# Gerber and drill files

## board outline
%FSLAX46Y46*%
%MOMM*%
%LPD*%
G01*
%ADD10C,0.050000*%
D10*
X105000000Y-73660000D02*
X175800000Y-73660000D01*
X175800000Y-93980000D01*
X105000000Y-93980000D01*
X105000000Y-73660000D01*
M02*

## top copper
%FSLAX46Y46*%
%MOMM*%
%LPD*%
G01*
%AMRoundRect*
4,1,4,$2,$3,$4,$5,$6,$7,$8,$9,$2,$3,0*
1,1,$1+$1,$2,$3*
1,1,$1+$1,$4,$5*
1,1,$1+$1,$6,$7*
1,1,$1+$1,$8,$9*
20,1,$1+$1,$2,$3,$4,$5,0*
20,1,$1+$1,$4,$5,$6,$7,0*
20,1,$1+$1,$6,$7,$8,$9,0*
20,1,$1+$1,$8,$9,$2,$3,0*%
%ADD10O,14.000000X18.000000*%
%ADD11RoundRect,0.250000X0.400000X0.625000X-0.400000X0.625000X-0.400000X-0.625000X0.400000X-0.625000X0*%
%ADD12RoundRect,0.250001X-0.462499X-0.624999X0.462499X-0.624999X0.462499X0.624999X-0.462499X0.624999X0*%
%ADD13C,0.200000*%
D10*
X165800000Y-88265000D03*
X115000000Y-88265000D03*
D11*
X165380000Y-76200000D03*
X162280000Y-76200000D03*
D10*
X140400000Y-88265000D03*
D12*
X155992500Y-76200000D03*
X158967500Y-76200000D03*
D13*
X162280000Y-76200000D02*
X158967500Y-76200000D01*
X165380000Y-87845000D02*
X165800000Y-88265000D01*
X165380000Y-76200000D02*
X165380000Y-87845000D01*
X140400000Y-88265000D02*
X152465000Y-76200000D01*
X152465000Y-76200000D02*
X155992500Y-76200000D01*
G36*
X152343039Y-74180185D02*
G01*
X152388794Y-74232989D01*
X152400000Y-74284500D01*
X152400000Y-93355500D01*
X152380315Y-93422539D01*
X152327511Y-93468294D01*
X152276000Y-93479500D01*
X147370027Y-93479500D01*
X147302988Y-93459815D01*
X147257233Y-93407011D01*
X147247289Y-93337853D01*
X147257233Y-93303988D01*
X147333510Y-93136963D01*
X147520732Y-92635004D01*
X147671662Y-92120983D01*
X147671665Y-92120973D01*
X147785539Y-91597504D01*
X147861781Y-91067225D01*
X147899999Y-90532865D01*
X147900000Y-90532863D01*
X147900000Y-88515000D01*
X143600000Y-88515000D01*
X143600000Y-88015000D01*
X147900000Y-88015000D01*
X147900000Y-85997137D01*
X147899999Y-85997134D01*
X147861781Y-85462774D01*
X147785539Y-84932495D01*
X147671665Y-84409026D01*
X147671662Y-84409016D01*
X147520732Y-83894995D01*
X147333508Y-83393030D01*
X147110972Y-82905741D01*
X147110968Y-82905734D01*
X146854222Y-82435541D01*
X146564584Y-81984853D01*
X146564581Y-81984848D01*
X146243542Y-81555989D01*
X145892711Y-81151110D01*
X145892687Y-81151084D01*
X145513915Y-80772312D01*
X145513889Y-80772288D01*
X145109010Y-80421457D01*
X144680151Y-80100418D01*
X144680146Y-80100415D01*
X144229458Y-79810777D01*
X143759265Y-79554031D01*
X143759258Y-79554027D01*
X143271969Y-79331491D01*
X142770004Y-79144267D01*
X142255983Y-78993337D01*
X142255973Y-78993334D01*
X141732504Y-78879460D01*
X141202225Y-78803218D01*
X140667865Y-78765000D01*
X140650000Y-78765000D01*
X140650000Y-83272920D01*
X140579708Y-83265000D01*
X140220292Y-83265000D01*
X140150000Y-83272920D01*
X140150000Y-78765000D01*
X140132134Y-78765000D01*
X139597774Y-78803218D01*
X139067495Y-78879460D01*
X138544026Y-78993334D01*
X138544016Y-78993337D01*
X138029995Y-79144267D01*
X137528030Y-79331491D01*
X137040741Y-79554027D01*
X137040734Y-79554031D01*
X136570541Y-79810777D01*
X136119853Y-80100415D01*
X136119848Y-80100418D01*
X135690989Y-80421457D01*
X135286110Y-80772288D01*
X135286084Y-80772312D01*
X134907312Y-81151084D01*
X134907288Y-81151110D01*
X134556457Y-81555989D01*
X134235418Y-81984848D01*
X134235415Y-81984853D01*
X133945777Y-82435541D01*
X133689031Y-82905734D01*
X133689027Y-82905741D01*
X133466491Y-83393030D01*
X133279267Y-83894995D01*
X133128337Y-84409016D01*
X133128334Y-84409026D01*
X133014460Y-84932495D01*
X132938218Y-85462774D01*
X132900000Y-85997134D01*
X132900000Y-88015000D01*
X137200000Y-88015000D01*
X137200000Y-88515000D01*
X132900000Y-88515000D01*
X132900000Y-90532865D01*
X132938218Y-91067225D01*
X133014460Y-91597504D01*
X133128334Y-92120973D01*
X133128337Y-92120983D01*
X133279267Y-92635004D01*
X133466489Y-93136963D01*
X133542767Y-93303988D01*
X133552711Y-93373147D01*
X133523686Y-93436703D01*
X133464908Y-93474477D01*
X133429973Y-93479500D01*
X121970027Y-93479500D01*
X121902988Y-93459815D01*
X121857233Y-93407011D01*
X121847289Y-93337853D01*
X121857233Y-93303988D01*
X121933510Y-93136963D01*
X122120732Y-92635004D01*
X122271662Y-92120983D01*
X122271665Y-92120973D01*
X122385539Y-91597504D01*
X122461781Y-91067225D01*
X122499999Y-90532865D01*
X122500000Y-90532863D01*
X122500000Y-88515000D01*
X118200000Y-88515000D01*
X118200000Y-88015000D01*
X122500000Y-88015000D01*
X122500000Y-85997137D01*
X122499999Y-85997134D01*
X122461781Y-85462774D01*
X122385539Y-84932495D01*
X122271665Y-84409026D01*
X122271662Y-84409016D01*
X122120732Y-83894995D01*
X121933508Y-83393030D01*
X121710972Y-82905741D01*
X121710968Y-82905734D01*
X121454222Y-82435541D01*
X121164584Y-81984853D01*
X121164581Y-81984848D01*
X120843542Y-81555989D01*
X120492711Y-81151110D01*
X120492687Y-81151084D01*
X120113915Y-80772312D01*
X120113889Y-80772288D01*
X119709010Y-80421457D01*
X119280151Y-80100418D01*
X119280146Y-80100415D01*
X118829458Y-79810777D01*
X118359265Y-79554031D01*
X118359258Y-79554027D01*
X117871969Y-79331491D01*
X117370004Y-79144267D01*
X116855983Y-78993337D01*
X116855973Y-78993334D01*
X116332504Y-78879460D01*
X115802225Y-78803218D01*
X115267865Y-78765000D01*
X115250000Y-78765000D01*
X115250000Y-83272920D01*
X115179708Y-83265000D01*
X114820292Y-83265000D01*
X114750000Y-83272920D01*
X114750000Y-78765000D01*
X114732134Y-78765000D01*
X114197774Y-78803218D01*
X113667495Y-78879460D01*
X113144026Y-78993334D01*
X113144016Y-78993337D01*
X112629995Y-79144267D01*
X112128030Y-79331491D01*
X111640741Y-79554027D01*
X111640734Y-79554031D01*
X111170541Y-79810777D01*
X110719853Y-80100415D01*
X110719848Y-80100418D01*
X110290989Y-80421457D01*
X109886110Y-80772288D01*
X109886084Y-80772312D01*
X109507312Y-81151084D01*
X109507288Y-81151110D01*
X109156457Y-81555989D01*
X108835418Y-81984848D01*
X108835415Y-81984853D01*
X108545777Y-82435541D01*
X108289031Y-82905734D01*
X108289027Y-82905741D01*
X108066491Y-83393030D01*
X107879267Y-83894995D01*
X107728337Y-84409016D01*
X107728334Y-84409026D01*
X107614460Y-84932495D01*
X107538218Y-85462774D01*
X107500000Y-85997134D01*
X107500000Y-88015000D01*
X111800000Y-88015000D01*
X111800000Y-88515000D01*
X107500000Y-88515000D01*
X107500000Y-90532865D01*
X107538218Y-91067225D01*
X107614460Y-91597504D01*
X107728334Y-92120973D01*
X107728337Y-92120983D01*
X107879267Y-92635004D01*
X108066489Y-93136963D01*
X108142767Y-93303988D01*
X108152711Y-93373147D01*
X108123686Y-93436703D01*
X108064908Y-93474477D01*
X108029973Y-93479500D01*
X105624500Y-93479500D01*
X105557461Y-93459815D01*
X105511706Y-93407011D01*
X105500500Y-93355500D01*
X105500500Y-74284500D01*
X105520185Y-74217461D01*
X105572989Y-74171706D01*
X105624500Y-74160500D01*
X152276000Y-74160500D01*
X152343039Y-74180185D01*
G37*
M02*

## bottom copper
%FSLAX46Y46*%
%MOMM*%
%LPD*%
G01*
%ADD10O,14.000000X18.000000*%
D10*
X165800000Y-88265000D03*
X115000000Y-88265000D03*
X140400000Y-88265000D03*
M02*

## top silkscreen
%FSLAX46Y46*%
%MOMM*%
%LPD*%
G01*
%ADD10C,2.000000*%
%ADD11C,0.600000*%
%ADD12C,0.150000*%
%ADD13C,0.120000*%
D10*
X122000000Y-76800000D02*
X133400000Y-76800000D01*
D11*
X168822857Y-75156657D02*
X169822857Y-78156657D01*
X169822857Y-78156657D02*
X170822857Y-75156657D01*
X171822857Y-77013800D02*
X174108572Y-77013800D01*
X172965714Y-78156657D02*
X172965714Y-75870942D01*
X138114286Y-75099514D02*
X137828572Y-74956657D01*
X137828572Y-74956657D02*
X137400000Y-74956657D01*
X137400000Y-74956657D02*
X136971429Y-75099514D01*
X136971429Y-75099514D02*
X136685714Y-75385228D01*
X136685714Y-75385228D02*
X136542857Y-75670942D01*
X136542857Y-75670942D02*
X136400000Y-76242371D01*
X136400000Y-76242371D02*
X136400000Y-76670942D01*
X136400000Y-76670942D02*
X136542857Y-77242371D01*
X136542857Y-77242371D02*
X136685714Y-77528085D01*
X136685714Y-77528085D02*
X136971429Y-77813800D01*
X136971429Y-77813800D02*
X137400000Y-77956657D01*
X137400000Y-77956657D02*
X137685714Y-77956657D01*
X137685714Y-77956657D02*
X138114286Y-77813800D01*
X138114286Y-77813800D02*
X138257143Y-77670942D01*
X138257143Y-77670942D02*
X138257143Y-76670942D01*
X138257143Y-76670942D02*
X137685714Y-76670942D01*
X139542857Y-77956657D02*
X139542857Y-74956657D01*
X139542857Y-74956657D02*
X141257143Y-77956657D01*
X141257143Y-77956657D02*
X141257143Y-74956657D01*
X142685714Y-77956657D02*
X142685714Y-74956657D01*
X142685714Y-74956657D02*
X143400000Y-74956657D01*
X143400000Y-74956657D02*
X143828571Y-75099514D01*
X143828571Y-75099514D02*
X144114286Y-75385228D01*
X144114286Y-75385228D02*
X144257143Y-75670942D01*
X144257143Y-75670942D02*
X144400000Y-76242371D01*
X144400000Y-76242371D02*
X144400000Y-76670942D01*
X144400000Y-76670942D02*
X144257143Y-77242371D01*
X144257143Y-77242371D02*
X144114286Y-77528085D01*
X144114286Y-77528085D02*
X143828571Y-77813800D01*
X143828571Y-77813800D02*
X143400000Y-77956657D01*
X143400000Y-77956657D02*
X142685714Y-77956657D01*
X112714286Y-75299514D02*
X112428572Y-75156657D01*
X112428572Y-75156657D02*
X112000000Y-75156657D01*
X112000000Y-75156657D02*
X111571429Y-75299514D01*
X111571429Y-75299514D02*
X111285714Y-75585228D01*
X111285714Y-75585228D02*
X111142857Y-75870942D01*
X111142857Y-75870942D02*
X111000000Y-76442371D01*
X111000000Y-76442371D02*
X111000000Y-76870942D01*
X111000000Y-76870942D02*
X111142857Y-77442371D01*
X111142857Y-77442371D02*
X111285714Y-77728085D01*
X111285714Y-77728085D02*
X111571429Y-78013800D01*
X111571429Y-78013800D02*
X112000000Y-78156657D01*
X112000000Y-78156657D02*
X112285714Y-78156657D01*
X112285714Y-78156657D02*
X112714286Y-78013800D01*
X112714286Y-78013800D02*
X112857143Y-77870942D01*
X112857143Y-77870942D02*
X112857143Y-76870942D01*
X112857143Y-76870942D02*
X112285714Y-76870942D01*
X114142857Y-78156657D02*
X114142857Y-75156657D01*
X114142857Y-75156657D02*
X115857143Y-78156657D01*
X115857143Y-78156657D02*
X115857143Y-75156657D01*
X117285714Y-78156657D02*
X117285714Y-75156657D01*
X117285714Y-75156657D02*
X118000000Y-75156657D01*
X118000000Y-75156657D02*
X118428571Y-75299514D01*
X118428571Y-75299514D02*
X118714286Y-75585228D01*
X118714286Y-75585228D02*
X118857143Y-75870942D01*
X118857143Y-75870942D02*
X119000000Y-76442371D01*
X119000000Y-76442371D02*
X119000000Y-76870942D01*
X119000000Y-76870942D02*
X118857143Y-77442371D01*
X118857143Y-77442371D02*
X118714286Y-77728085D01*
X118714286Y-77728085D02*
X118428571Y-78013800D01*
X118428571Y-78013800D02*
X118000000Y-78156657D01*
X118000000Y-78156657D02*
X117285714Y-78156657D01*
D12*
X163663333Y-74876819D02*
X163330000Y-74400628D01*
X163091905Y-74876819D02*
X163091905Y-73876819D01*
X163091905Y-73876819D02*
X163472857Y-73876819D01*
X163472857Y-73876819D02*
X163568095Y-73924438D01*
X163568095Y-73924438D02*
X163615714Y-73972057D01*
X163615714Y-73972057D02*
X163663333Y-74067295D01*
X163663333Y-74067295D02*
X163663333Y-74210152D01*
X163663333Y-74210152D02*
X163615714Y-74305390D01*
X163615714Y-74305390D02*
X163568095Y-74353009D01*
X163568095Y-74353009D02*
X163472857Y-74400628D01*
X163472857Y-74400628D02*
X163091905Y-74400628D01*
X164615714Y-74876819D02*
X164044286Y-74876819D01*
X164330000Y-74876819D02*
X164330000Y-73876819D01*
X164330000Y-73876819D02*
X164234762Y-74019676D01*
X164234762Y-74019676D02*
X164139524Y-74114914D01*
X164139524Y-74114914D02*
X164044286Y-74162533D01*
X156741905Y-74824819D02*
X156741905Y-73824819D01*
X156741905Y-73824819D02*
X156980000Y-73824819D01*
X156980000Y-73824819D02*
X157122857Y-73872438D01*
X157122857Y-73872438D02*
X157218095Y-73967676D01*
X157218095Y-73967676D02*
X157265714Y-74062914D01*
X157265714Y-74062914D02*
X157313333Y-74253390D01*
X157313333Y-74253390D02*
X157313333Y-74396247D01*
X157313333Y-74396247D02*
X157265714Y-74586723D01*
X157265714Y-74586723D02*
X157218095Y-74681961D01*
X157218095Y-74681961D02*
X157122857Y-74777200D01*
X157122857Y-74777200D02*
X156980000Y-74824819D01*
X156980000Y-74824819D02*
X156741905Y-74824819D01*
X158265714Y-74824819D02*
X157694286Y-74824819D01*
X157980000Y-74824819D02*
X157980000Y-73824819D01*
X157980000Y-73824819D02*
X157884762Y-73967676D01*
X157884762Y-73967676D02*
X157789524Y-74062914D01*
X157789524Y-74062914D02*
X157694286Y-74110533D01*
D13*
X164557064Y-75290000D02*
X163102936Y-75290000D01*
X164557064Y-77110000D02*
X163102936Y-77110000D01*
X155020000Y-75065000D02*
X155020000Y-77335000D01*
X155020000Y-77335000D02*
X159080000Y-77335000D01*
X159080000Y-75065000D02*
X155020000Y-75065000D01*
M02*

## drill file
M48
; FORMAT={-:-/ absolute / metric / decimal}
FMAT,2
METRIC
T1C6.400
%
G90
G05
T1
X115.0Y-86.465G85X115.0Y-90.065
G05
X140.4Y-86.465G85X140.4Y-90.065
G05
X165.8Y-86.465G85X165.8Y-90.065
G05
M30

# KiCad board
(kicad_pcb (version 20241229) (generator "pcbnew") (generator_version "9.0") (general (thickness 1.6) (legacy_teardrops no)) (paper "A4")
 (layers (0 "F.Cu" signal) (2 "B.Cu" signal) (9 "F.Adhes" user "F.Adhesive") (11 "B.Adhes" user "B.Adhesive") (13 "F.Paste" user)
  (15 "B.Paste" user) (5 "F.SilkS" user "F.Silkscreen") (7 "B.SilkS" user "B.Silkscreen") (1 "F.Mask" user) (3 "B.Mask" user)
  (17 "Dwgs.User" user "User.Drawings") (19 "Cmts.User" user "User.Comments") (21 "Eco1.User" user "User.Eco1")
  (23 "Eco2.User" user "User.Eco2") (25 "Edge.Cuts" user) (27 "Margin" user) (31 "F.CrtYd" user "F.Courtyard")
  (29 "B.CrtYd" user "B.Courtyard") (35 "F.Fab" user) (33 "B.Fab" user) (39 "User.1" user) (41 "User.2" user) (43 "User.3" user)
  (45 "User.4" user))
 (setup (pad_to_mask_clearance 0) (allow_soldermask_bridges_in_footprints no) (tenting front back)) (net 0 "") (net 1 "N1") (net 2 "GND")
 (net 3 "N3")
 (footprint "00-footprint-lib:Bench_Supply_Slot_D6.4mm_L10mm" (layer "F.Cu") (at 165.8 88.265)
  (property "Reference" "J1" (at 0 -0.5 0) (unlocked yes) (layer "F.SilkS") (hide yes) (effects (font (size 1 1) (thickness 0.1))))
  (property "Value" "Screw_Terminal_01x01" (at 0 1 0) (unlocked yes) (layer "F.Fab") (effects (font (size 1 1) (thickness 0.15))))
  (pad "1" thru_hole oval (at 0 0) (size 14 18) (drill oval 6.4 10) (layers "*.Cu" "*.Mask") (remove_unused_layers no) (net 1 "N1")))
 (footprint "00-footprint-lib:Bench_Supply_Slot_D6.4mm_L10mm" (layer "F.Cu") (at 115 88.265)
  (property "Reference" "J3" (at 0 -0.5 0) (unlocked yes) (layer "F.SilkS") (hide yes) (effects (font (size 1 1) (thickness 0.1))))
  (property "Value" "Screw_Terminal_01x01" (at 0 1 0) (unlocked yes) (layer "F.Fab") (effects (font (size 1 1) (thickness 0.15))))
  (pad "1" thru_hole oval (at 0 0) (size 14 18) (drill oval 6.4 10) (layers "*.Cu" "*.Mask") (remove_unused_layers no) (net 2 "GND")))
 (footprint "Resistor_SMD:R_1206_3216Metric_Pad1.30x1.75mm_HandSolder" (layer "F.Cu") (at 163.83 76.2 180)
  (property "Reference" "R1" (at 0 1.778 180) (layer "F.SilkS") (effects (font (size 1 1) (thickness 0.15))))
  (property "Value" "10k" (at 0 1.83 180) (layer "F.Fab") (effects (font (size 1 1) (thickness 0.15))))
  (fp_line (start -0.727064 0.91) (end 0.727064 0.91) (stroke (width 0.12) (type solid)) (layer "F.SilkS"))
  (fp_line (start -0.727064 -0.91) (end 0.727064 -0.91) (stroke (width 0.12) (type solid)) (layer "F.SilkS"))
  (pad "1" smd roundrect (at -1.55 0 180) (size 1.3 1.75) (layers "F.Cu" "F.Mask" "F.Paste") (roundrect_rratio 0.192308) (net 1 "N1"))
  (pad "2" smd roundrect (at 1.55 0 180) (size 1.3 1.75) (layers "F.Cu" "F.Mask" "F.Paste") (roundrect_rratio 0.192308) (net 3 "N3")))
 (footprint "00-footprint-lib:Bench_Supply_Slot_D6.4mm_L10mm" (layer "F.Cu") (at 140.4 88.265)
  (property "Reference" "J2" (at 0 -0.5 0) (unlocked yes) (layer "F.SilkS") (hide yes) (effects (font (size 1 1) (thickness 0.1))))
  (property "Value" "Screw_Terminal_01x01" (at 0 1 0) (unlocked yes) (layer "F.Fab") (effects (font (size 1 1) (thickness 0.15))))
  (pad "1" thru_hole oval (at 0 0) (size 14 18) (drill oval 6.4 10) (layers "*.Cu" "*.Mask") (remove_unused_layers no) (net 2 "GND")))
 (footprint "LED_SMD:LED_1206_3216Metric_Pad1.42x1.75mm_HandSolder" (layer "F.Cu") (at 157.48 76.2)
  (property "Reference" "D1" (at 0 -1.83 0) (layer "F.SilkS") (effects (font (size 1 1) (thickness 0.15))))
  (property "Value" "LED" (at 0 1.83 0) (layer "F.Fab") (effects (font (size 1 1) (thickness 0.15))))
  (fp_line (start -2.46 -1.135) (end -2.46 1.135) (stroke (width 0.12) (type solid)) (layer "F.SilkS"))
  (fp_line (start -2.46 1.135) (end 1.6 1.135) (stroke (width 0.12) (type solid)) (layer "F.SilkS"))
  (fp_line (start 1.6 -1.135) (end -2.46 -1.135) (stroke (width 0.12) (type solid)) (layer "F.SilkS"))
  (pad "1" smd roundrect (at -1.4875 0) (size 1.425 1.75) (layers "F.Cu" "F.Mask" "F.Paste") (roundrect_rratio 0.175439) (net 2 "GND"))
  (pad "2" smd roundrect (at 1.4875 0) (size 1.425 1.75) (layers "F.Cu" "F.Mask" "F.Paste") (roundrect_rratio 0.175439) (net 3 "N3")))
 (gr_line (start 122 76.8) (end 133.4 76.8) (stroke (width 2) (type solid)) (layer "F.SilkS"))
 (gr_rect (start 105 73.66) (end 175.8 93.98) (stroke (width 0.05) (type solid)) (fill no) (layer "Edge.Cuts"))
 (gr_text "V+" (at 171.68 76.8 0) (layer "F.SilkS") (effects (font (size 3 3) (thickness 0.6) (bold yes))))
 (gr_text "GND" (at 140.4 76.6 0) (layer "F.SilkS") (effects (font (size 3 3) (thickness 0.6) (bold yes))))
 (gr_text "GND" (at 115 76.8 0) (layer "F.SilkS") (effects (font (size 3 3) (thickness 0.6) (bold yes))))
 (segment (start 162.28 76.2) (end 158.9675 76.2) (width 0.2) (layer "F.Cu") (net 3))
 (segment (start 165.38 87.845) (end 165.8 88.265) (width 0.2) (layer "F.Cu") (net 1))
 (segment (start 165.38 76.2) (end 165.38 87.845) (width 0.2) (layer "F.Cu") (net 1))
 (segment (start 140.4 88.265) (end 152.465 76.2) (width 0.2) (layer "F.Cu") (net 2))
 (segment (start 152.465 76.2) (end 155.9925 76.2) (width 0.2) (layer "F.Cu") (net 2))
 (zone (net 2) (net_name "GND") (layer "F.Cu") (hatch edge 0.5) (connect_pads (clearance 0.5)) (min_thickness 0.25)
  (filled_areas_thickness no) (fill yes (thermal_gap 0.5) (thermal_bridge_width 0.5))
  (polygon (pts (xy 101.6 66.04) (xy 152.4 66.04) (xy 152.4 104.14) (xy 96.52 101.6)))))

